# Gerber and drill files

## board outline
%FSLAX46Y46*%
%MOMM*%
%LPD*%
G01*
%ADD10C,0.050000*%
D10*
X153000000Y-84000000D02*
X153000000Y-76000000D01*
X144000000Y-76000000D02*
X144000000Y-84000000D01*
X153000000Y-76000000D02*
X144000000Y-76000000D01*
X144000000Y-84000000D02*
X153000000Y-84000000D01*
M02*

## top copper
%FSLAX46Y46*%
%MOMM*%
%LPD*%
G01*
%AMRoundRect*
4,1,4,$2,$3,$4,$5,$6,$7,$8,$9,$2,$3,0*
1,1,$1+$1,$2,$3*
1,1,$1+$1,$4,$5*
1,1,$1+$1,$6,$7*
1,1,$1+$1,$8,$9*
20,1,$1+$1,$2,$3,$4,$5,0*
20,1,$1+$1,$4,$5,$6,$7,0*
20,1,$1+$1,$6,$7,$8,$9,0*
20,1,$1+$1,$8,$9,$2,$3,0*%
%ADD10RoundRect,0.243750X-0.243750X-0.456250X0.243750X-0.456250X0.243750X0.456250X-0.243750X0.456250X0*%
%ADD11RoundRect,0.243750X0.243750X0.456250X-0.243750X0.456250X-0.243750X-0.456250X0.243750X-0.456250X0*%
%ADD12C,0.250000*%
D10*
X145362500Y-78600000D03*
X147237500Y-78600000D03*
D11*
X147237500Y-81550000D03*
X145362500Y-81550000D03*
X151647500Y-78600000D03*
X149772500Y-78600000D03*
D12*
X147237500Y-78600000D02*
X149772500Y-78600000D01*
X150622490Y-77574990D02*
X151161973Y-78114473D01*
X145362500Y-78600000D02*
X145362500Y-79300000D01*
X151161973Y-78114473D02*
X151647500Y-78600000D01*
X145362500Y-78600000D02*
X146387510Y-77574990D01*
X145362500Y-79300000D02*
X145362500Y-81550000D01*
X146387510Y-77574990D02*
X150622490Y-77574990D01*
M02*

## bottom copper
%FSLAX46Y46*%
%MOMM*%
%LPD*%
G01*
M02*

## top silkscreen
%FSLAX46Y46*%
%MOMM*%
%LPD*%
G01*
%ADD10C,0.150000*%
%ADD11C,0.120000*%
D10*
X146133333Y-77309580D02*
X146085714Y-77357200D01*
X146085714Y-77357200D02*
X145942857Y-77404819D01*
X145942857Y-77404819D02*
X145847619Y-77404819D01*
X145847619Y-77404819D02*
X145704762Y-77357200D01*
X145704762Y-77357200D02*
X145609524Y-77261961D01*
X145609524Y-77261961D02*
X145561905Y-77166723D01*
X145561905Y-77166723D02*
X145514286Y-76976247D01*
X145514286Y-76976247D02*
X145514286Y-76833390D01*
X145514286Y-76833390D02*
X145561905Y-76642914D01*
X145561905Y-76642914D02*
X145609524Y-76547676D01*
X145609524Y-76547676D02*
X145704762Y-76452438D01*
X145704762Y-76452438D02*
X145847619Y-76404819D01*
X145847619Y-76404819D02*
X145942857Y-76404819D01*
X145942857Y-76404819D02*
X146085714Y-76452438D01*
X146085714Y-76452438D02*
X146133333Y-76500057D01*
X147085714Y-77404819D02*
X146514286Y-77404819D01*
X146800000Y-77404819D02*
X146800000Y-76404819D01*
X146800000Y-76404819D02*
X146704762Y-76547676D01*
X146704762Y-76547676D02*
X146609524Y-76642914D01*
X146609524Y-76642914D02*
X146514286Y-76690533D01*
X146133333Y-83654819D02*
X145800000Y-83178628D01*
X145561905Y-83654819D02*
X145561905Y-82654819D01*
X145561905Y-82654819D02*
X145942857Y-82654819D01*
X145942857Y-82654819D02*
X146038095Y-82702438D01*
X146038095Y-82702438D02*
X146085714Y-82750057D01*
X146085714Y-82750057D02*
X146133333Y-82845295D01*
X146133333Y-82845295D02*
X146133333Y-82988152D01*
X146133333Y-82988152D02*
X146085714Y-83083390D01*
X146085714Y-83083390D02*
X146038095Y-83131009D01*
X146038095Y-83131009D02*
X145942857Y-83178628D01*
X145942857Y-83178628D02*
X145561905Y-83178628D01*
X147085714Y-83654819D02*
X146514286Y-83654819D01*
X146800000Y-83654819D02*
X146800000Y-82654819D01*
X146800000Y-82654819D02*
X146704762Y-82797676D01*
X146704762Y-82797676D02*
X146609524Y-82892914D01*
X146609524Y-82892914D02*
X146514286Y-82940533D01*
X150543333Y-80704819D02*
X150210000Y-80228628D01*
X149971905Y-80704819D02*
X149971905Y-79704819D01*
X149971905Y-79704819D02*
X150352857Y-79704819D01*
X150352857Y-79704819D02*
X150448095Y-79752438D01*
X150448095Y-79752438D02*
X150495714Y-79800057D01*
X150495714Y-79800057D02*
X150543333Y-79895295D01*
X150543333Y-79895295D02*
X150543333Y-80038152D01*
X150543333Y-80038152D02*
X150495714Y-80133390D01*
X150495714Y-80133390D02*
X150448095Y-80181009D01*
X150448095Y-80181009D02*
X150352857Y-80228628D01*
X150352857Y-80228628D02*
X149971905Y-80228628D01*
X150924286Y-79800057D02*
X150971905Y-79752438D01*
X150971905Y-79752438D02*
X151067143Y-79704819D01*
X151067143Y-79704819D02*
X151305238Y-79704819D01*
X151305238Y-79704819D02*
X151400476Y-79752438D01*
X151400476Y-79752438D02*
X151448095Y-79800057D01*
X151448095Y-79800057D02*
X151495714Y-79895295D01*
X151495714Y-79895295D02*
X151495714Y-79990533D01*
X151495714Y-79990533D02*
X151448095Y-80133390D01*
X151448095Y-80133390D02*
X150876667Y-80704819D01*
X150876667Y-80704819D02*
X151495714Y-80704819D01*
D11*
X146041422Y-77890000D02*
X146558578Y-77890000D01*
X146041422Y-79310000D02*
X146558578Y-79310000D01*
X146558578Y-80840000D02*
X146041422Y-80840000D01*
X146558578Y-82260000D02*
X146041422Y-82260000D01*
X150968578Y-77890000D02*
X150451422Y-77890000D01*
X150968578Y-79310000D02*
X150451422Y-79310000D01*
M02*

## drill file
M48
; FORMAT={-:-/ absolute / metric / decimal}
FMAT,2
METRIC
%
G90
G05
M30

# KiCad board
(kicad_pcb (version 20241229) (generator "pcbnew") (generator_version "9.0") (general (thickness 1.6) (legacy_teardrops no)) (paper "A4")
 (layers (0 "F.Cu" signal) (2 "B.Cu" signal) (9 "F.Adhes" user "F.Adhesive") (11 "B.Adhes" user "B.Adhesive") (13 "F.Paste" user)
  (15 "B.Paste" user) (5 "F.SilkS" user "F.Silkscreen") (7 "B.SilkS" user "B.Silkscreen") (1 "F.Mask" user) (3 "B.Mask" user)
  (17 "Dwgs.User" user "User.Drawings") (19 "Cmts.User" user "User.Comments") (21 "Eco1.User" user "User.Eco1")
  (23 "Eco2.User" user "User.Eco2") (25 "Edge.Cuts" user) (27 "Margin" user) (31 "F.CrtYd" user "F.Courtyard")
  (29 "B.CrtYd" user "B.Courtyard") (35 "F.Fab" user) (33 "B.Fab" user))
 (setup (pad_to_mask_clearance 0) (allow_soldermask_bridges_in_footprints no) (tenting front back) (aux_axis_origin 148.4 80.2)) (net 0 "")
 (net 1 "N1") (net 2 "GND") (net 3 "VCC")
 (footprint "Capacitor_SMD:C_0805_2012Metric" (layer "F.Cu") (at 146.3 78.6)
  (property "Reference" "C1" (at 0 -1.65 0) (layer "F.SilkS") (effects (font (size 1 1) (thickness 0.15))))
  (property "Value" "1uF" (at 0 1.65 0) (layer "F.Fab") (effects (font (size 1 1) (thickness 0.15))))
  (fp_line (start -0.258578 -0.71) (end 0.258578 -0.71) (stroke (width 0.12) (type solid)) (layer "F.SilkS"))
  (fp_line (start -0.258578 0.71) (end 0.258578 0.71) (stroke (width 0.12) (type solid)) (layer "F.SilkS"))
  (pad "1" smd roundrect (at -0.9375 0) (size 0.975 1.4) (layers "F.Cu" "F.Mask" "F.Paste") (roundrect_rratio 0.25) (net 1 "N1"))
  (pad "2" smd roundrect (at 0.9375 0) (size 0.975 1.4) (layers "F.Cu" "F.Mask" "F.Paste") (roundrect_rratio 0.25) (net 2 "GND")))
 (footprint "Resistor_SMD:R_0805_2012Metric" (layer "F.Cu") (at 146.3 81.55 180)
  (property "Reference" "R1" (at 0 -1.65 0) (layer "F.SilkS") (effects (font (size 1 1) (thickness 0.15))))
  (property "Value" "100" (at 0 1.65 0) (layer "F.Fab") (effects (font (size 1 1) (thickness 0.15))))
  (fp_line (start -0.258578 0.71) (end 0.258578 0.71) (stroke (width 0.12) (type solid)) (layer "F.SilkS"))
  (fp_line (start -0.258578 -0.71) (end 0.258578 -0.71) (stroke (width 0.12) (type solid)) (layer "F.SilkS"))
  (pad "1" smd roundrect (at -0.9375 0 180) (size 0.975 1.4) (layers "F.Cu" "F.Mask" "F.Paste") (roundrect_rratio 0.25) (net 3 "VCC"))
  (pad "2" smd roundrect (at 0.9375 0 180) (size 0.975 1.4) (layers "F.Cu" "F.Mask" "F.Paste") (roundrect_rratio 0.25) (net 1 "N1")))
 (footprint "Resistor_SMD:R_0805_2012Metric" (layer "F.Cu") (at 150.71 78.6 180)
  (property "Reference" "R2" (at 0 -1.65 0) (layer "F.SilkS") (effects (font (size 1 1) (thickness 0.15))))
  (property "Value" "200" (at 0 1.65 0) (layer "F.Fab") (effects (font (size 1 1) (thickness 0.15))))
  (fp_line (start -0.258578 0.71) (end 0.258578 0.71) (stroke (width 0.12) (type solid)) (layer "F.SilkS"))
  (fp_line (start -0.258578 -0.71) (end 0.258578 -0.71) (stroke (width 0.12) (type solid)) (layer "F.SilkS"))
  (pad "1" smd roundrect (at -0.9375 0 180) (size 0.975 1.4) (layers "F.Cu" "F.Mask" "F.Paste") (roundrect_rratio 0.25) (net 1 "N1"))
  (pad "2" smd roundrect (at 0.9375 0 180) (size 0.975 1.4) (layers "F.Cu" "F.Mask" "F.Paste") (roundrect_rratio 0.25) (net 2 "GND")))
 (gr_line (start 153 84) (end 153 76) (stroke (width 0.05) (type solid)) (layer "Edge.Cuts"))
 (gr_line (start 144 76) (end 144 84) (stroke (width 0.05) (type solid)) (layer "Edge.Cuts"))
 (gr_line (start 153 76) (end 144 76) (stroke (width 0.05) (type solid)) (layer "Edge.Cuts"))
 (gr_line (start 144 84) (end 153 84) (stroke (width 0.05) (type solid)) (layer "Edge.Cuts"))
 (segment (start 147.2375 78.6) (end 149.7725 78.6) (width 0.25) (layer "F.Cu") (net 2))
 (segment (start 150.62249 77.57499) (end 151.161973 78.114473) (width 0.25) (layer "F.Cu") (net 1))
 (segment (start 145.3625 78.6) (end 145.3625 79.3) (width 0.25) (layer "F.Cu") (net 1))
 (segment (start 151.161973 78.114473) (end 151.6475 78.6) (width 0.25) (layer "F.Cu") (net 1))
 (segment (start 145.3625 78.6) (end 146.38751 77.57499) (width 0.25) (layer "F.Cu") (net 1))
 (segment (start 145.3625 79.3) (end 145.3625 81.55) (width 0.25) (layer "F.Cu") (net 1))
 (segment (start 146.38751 77.57499) (end 150.62249 77.57499) (width 0.25) (layer "F.Cu") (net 1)))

